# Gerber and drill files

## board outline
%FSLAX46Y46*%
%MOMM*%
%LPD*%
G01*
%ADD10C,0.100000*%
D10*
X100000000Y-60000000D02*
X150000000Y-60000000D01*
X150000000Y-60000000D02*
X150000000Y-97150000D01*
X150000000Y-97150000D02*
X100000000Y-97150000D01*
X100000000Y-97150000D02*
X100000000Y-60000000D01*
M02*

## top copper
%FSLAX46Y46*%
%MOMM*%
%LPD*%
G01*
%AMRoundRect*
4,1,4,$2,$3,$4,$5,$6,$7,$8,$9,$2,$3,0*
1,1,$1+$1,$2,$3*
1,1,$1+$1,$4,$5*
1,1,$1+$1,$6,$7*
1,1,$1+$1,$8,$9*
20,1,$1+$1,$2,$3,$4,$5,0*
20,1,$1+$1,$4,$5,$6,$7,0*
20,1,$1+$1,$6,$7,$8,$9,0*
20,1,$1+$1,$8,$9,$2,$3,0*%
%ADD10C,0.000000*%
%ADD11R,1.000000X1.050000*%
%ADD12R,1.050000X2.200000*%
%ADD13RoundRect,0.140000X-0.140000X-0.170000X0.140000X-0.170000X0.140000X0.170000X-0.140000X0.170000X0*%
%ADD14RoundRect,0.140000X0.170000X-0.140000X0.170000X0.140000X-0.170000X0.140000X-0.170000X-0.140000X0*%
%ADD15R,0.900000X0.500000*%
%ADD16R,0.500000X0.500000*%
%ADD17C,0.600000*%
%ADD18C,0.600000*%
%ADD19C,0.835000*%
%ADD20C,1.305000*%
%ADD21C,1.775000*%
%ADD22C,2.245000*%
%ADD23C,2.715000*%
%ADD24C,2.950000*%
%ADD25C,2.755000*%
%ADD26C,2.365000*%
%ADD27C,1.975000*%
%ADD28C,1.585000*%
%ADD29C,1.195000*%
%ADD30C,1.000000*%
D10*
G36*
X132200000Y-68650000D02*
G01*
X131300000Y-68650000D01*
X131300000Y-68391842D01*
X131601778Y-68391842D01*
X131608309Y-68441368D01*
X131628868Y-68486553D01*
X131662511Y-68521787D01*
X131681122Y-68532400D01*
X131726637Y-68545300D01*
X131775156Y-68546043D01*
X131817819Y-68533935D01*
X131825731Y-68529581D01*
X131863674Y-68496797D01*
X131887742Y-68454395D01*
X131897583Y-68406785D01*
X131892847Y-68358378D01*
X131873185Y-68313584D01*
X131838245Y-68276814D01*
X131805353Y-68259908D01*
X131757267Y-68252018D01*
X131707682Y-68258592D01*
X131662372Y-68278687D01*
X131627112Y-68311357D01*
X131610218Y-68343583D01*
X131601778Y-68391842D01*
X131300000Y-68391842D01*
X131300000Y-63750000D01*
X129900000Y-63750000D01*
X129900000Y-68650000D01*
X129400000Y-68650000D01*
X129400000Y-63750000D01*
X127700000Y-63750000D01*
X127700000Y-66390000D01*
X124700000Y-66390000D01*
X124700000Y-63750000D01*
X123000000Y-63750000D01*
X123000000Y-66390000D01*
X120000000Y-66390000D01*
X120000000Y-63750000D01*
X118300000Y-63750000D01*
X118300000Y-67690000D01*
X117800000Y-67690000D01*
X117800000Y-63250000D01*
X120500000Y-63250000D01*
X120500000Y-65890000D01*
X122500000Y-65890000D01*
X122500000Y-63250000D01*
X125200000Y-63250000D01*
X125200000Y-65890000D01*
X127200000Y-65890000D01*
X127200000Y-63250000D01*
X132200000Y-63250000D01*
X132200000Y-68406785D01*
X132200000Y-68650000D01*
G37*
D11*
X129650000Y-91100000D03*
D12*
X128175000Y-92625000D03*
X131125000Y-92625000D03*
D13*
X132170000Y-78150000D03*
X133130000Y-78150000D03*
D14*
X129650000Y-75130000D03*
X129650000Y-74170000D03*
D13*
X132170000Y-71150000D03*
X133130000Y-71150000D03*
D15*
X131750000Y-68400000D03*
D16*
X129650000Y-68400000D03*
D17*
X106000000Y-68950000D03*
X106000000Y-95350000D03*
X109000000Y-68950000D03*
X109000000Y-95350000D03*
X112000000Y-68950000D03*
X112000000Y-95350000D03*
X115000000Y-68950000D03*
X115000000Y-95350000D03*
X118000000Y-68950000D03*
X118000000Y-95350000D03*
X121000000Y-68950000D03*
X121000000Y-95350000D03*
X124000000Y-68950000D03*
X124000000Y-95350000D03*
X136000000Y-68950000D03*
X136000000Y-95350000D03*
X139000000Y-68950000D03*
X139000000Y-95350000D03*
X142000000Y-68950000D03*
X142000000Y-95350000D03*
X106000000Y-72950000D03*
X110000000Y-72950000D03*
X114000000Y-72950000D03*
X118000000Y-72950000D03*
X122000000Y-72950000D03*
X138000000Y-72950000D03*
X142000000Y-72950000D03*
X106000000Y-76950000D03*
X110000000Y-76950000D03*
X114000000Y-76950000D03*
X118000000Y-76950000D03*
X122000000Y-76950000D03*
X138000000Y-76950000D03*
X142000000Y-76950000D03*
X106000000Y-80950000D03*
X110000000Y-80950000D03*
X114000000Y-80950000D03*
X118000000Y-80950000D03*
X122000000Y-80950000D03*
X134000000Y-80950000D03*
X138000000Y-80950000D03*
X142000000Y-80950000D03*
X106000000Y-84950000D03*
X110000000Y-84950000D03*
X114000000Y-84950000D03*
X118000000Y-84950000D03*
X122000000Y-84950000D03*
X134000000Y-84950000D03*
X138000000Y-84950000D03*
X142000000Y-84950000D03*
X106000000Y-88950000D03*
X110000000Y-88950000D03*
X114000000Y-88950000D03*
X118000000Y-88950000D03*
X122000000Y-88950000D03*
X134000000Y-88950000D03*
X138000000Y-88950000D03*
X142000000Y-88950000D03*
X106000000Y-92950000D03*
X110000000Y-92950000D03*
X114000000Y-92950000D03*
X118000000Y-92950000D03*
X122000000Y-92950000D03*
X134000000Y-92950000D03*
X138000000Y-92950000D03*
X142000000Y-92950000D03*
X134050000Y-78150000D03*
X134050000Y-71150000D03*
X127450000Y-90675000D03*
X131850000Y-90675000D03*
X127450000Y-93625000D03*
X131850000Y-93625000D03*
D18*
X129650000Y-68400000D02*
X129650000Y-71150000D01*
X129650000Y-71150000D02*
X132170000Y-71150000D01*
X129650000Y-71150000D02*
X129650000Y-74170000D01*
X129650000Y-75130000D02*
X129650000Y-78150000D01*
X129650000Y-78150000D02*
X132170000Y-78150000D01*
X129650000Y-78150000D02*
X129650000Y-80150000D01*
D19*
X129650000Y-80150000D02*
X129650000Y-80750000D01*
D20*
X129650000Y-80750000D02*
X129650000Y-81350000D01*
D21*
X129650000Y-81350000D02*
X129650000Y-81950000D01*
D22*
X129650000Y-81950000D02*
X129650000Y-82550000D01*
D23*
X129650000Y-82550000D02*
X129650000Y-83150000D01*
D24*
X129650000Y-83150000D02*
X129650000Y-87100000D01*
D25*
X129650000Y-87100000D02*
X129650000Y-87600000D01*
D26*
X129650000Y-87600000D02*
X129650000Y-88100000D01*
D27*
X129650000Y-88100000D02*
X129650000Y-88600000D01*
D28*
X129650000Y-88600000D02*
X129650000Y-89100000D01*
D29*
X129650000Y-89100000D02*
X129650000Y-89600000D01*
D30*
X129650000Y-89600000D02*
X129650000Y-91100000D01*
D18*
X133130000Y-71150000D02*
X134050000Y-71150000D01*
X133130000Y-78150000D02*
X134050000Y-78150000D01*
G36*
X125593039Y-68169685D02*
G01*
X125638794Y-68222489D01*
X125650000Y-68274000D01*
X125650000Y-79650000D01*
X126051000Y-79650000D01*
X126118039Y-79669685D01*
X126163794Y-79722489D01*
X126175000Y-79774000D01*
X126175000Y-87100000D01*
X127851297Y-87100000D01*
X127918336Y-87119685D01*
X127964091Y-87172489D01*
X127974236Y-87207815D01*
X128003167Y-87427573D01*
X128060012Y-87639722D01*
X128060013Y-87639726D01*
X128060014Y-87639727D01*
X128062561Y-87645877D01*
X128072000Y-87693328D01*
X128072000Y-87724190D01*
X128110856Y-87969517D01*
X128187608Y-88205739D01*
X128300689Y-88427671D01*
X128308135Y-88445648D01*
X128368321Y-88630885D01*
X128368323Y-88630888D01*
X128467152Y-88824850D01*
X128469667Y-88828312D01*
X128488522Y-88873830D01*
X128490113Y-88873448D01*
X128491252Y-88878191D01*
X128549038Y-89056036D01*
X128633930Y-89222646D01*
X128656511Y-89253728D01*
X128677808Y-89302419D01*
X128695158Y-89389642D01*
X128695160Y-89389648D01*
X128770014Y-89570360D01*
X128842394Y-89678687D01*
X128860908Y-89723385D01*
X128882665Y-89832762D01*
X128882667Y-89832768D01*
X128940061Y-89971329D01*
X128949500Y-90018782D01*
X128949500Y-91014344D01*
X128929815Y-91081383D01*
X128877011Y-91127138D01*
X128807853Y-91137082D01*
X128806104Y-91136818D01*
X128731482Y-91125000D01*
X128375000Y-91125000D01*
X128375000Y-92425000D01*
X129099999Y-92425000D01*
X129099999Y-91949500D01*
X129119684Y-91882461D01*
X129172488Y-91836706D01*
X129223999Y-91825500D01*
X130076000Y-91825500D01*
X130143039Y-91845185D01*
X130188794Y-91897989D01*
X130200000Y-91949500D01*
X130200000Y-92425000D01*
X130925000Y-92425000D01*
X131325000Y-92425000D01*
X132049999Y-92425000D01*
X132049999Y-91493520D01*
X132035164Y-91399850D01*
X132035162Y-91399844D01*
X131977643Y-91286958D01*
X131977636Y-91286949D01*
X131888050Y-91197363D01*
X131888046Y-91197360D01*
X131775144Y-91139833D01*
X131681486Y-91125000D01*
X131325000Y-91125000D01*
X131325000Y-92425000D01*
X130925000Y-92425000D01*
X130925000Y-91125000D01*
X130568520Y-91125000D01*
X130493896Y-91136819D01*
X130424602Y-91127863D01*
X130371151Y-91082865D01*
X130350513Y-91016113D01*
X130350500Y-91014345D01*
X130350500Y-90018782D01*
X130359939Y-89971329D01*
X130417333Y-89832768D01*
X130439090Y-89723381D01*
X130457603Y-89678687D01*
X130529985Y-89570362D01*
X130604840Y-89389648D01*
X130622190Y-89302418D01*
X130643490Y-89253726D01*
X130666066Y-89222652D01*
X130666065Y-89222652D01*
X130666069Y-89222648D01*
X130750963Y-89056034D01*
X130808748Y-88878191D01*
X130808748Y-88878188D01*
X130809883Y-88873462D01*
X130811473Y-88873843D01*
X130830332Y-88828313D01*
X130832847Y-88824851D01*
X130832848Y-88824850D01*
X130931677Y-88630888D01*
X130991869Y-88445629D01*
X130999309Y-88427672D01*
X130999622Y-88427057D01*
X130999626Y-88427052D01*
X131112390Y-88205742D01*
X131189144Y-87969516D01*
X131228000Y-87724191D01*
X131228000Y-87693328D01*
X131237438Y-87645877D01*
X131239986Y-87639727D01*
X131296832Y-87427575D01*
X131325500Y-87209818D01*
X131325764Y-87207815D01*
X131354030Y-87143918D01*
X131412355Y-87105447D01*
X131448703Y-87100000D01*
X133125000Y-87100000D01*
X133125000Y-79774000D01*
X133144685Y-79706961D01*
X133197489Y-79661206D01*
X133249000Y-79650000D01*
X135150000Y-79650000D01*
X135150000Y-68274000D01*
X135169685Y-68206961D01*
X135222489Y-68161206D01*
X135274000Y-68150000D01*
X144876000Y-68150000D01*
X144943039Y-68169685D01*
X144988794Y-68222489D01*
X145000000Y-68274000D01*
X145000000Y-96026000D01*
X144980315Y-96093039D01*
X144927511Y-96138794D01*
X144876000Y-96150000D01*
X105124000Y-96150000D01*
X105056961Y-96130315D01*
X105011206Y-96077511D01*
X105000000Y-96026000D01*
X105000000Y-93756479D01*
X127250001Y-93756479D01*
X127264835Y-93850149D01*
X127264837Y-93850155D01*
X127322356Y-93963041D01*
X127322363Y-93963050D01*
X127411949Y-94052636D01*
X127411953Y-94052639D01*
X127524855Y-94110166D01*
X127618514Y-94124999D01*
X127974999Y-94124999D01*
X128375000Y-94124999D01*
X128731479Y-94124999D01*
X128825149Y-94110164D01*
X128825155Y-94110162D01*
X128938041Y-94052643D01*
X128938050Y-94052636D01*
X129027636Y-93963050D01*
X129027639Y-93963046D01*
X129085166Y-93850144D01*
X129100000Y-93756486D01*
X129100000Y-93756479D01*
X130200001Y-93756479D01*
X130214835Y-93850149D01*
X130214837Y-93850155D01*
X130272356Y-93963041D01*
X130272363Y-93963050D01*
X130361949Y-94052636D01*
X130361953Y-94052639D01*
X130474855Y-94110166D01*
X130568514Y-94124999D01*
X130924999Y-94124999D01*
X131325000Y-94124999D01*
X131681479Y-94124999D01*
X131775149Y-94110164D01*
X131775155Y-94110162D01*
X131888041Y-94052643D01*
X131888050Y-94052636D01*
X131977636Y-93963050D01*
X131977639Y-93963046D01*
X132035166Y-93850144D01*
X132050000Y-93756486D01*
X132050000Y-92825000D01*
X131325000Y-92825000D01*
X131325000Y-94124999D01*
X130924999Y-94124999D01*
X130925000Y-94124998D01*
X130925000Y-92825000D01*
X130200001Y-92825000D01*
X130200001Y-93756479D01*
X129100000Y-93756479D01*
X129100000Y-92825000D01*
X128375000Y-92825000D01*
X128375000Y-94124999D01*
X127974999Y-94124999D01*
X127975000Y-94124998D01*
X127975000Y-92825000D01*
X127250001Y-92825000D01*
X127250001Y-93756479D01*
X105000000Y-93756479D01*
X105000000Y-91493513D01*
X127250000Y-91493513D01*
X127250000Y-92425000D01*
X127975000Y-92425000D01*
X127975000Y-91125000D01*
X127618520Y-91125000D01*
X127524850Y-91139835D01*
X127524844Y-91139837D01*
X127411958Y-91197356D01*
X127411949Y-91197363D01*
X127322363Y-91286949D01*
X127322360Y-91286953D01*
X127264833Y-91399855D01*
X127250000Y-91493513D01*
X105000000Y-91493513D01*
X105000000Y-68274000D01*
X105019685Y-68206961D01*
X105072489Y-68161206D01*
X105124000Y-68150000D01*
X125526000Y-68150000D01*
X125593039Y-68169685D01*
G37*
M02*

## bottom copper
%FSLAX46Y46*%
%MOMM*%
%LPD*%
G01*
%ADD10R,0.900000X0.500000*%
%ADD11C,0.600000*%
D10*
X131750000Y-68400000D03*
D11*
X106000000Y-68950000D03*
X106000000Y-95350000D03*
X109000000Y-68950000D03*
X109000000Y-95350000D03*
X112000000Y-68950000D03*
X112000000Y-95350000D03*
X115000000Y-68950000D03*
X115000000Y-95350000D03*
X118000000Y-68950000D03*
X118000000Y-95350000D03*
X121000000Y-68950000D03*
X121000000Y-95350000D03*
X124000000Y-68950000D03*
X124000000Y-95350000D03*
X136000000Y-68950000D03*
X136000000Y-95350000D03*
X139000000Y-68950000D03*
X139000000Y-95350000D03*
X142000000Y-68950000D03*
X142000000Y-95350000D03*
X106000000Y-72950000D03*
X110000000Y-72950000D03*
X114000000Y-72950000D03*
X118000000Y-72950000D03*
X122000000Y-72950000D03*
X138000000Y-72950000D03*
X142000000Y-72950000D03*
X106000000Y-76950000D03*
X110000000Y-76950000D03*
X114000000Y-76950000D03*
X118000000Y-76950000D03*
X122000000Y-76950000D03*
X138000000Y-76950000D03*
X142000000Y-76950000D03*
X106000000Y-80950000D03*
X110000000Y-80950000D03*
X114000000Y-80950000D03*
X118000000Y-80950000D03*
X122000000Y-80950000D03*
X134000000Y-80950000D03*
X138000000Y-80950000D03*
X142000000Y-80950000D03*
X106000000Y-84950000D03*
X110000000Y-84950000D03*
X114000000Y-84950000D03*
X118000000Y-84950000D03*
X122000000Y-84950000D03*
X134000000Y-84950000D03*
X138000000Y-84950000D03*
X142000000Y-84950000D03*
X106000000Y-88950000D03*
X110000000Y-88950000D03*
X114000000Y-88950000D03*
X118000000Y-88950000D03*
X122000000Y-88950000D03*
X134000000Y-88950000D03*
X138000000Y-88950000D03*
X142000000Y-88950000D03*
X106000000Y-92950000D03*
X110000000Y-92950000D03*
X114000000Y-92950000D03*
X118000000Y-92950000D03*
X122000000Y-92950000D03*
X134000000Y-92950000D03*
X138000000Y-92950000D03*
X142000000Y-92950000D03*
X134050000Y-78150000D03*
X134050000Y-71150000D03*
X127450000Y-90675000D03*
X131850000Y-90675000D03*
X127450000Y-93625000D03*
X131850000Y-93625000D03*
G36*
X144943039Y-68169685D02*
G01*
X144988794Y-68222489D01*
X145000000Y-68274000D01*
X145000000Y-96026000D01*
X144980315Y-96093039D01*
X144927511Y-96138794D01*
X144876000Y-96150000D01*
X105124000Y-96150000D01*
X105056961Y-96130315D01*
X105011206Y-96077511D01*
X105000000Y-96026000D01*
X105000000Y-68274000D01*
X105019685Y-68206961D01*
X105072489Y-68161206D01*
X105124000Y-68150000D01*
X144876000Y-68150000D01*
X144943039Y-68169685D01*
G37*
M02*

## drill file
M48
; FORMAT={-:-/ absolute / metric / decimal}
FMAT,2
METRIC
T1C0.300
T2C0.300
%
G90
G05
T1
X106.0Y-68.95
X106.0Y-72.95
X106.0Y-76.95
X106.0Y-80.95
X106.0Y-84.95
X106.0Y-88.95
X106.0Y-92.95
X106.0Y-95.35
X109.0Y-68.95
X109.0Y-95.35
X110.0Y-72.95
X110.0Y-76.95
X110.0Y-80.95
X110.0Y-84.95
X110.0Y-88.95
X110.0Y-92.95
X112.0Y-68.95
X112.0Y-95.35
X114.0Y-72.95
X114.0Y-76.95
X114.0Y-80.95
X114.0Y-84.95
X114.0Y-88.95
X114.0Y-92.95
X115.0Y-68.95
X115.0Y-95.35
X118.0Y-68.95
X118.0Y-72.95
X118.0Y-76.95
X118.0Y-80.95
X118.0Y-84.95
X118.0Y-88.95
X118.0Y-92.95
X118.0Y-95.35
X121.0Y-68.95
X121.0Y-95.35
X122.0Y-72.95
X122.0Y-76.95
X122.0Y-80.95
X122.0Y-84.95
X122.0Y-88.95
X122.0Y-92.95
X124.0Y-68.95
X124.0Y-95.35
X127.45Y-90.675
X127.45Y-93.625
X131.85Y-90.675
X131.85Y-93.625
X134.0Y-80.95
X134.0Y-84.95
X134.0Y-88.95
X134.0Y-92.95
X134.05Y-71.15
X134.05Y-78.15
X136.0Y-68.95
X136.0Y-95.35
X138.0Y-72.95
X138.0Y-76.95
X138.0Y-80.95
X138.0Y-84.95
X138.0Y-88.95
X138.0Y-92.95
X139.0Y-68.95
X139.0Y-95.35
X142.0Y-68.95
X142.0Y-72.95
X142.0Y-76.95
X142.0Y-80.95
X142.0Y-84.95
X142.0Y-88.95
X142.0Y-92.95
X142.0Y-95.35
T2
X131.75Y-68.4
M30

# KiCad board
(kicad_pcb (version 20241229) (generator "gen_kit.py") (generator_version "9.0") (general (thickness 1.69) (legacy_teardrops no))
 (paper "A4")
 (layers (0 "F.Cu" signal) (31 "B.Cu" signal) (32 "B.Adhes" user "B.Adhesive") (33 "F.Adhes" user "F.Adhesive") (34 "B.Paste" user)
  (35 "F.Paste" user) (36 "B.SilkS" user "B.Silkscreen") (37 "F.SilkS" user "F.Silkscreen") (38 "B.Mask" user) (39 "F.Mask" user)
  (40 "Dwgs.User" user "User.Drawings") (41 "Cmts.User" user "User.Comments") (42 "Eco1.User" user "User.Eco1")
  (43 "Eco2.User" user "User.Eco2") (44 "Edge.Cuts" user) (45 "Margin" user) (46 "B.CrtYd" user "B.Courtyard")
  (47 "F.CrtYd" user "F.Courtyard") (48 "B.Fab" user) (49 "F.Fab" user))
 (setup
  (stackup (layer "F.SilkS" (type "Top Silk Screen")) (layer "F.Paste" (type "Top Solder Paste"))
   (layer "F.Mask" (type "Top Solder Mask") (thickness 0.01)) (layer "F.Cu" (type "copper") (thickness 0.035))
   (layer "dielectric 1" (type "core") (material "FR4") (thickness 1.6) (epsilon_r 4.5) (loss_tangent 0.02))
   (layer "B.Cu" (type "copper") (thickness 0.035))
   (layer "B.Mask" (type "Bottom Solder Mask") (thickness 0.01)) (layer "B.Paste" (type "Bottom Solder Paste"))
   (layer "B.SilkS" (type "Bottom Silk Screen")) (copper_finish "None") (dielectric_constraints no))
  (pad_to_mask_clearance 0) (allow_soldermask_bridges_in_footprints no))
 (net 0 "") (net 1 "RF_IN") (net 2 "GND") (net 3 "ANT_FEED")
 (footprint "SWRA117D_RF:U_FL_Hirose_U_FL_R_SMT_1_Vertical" (layer "F.Cu") (at 129.65 92.15 270)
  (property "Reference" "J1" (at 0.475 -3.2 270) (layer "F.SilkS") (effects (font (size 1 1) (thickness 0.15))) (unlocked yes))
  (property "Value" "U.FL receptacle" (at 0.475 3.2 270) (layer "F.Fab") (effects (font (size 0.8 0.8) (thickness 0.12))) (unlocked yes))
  (pad "1" smd rect (at -1.05 0 270) (size 1.05 1) (layers "F.Cu" "F.Paste" "F.Mask") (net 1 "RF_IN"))
  (pad "2" smd rect (at 0.475 1.475 270) (size 2.2 1.05) (layers "F.Cu" "F.Paste" "F.Mask") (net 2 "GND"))
  (pad "2" smd rect (at 0.475 -1.475 270) (size 2.2 1.05) (layers "F.Cu" "F.Paste" "F.Mask") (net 2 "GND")))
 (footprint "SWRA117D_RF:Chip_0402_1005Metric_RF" (layer "F.Cu") (at 132.65 78.15)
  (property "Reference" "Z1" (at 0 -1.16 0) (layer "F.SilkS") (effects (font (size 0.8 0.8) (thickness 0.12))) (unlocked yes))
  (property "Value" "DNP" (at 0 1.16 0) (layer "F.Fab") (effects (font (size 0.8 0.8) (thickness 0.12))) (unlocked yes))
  (pad "1" smd roundrect (at -0.48 0) (size 0.56 0.62) (layers "F.Cu" "F.Paste" "F.Mask") (roundrect_rratio 0.25) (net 1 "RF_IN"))
  (pad "2" smd roundrect (at 0.48 0) (size 0.56 0.62) (layers "F.Cu" "F.Paste" "F.Mask") (roundrect_rratio 0.25) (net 2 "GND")))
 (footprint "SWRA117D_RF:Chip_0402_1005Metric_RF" (layer "F.Cu") (at 129.65 74.65 90)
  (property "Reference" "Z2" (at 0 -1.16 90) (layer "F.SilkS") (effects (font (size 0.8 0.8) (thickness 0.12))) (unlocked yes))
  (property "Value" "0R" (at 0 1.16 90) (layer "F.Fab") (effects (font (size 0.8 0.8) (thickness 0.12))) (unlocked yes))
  (pad "1" smd roundrect (at -0.48 0 90) (size 0.56 0.62) (layers "F.Cu" "F.Paste" "F.Mask") (roundrect_rratio 0.25) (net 1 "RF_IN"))
  (pad "2" smd roundrect (at 0.48 0 90) (size 0.56 0.62) (layers "F.Cu" "F.Paste" "F.Mask") (roundrect_rratio 0.25) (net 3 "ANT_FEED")))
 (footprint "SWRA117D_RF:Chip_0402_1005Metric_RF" (layer "F.Cu") (at 132.65 71.15)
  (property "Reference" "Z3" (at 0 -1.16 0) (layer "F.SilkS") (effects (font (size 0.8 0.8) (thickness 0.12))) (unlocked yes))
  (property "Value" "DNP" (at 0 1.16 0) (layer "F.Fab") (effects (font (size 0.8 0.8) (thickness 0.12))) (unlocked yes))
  (pad "1" smd roundrect (at -0.48 0) (size 0.56 0.62) (layers "F.Cu" "F.Paste" "F.Mask") (roundrect_rratio 0.25) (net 3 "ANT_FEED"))
  (pad "2" smd roundrect (at 0.48 0) (size 0.56 0.62) (layers "F.Cu" "F.Paste" "F.Mask") (roundrect_rratio 0.25) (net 2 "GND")))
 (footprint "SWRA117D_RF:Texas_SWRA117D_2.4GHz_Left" (layer "F.Cu") (at 129.65 68.4)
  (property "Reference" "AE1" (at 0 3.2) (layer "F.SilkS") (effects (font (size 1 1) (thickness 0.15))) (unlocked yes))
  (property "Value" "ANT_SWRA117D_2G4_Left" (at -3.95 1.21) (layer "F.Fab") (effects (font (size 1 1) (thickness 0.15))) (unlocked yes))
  (fp_poly
   (pts (xy -2.45 -2.51) (xy -4.45 -2.51) (xy -4.45 -5.15) (xy -7.15 -5.15) (xy -7.15 -2.51) (xy -9.15 -2.51) (xy -9.15 -5.15)
    (xy -11.85 -5.15) (xy -11.85 -0.71) (xy -11.35 -0.71) (xy -11.35 -4.65) (xy -9.65 -4.65) (xy -9.65 -2.01) (xy -6.65 -2.01)
    (xy -6.65 -4.65) (xy -4.95 -4.65) (xy -4.95 -2.01) (xy -1.95 -2.01) (xy -1.95 -4.65) (xy -0.25 -4.65) (xy -0.25 0.25) (xy 0.25 0.25)
    (xy 0.25 -4.65) (xy 1.65 -4.65) (xy 1.65 0.25) (xy 2.55 0.25) (xy 2.55 0.006785) (xy 2.247583 0.006785) (xy 2.237742 0.054395)
    (xy 2.213674 0.096797) (xy 2.175731 0.129581) (xy 2.167819 0.133935) (xy 2.125156 0.146043) (xy 2.076637 0.1453) (xy 2.031122 0.1324)
    (xy 2.012511 0.121787) (xy 1.978868 0.086553) (xy 1.958309 0.041368) (xy 1.951778 -0.008158) (xy 1.960218 -0.056417)
    (xy 1.977112 -0.088643) (xy 2.012372 -0.121313) (xy 2.057682 -0.141408) (xy 2.107267 -0.147982) (xy 2.155353 -0.140092)
    (xy 2.188245 -0.123186) (xy 2.223185 -0.086416) (xy 2.242847 -0.041622) (xy 2.247583 0.006785) (xy 2.55 0.006785) (xy 2.55 -5.15)
    (xy -2.45 -5.15) (xy -2.45 -2.51))
   (stroke (width 0) (type solid)) (fill yes) (layer "F.Cu"))
  (pad "2" thru_hole rect (at 2.1 0) (size 0.9 0.5) (drill 0.3) (layers "*.Cu") (zone_connect 2) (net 2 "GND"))
  (pad "1" smd rect (at 0 0) (size 0.5 0.5) (layers "F.Cu") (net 3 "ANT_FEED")))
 (gr_line (start 100 60) (end 150 60) (stroke (width 0.1) (type solid)) (layer "Edge.Cuts"))
 (gr_line (start 150 60) (end 150 97.15) (stroke (width 0.1) (type solid)) (layer "Edge.Cuts"))
 (gr_line (start 150 97.15) (end 100 97.15) (stroke (width 0.1) (type solid)) (layer "Edge.Cuts"))
 (gr_line (start 100 97.15) (end 100 60) (stroke (width 0.1) (type solid)) (layer "Edge.Cuts"))
 (segment (start 129.65 68.4) (end 129.65 71.15) (width 0.6) (layer "F.Cu") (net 3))
 (segment (start 129.65 71.15) (end 132.17 71.15) (width 0.6) (layer "F.Cu") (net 3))
 (segment (start 129.65 71.15) (end 129.65 74.17) (width 0.6) (layer "F.Cu") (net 3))
 (segment (start 129.65 75.13) (end 129.65 78.15) (width 0.6) (layer "F.Cu") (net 1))
 (segment (start 129.65 78.15) (end 132.17 78.15) (width 0.6) (layer "F.Cu") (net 1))
 (segment (start 129.65 78.15) (end 129.65 80.15) (width 0.6) (layer "F.Cu") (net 1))
 (segment (start 129.65 80.15) (end 129.65 80.75) (width 0.835) (layer "F.Cu") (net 1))
 (segment (start 129.65 80.75) (end 129.65 81.35) (width 1.305) (layer "F.Cu") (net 1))
 (segment (start 129.65 81.35) (end 129.65 81.95) (width 1.775) (layer "F.Cu") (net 1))
 (segment (start 129.65 81.95) (end 129.65 82.55) (width 2.245) (layer "F.Cu") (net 1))
 (segment (start 129.65 82.55) (end 129.65 83.15) (width 2.715) (layer "F.Cu") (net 1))
 (segment (start 129.65 83.15) (end 129.65 87.1) (width 2.95) (layer "F.Cu") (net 1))
 (segment (start 129.65 87.1) (end 129.65 87.6) (width 2.755) (layer "F.Cu") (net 1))
 (segment (start 129.65 87.6) (end 129.65 88.1) (width 2.365) (layer "F.Cu") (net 1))
 (segment (start 129.65 88.1) (end 129.65 88.6) (width 1.975) (layer "F.Cu") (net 1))
 (segment (start 129.65 88.6) (end 129.65 89.1) (width 1.585) (layer "F.Cu") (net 1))
 (segment (start 129.65 89.1) (end 129.65 89.6) (width 1.195) (layer "F.Cu") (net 1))
 (segment (start 129.65 89.6) (end 129.65 91.1) (width 1) (layer "F.Cu") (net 1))
 (segment (start 133.13 71.15) (end 134.05 71.15) (width 0.6) (layer "F.Cu") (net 2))
 (segment (start 133.13 78.15) (end 134.05 78.15) (width 0.6) (layer "F.Cu") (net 2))
 (via (at 106 68.95) (size 0.6) (drill 0.3) (layers "F.Cu" "B.Cu") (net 2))
 (via (at 106 95.35) (size 0.6) (drill 0.3) (layers "F.Cu" "B.Cu") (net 2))
 (via (at 109 68.95) (size 0.6) (drill 0.3) (layers "F.Cu" "B.Cu") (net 2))
 (via (at 109 95.35) (size 0.6) (drill 0.3) (layers "F.Cu" "B.Cu") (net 2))
 (via (at 112 68.95) (size 0.6) (drill 0.3) (layers "F.Cu" "B.Cu") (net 2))
 (via (at 112 95.35) (size 0.6) (drill 0.3) (layers "F.Cu" "B.Cu") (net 2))
 (via (at 115 68.95) (size 0.6) (drill 0.3) (layers "F.Cu" "B.Cu") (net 2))
 (via (at 115 95.35) (size 0.6) (drill 0.3) (layers "F.Cu" "B.Cu") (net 2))
 (via (at 118 68.95) (size 0.6) (drill 0.3) (layers "F.Cu" "B.Cu") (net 2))
 (via (at 118 95.35) (size 0.6) (drill 0.3) (layers "F.Cu" "B.Cu") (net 2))
 (via (at 121 68.95) (size 0.6) (drill 0.3) (layers "F.Cu" "B.Cu") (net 2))
 (via (at 121 95.35) (size 0.6) (drill 0.3) (layers "F.Cu" "B.Cu") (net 2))
 (via (at 124 68.95) (size 0.6) (drill 0.3) (layers "F.Cu" "B.Cu") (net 2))
 (via (at 124 95.35) (size 0.6) (drill 0.3) (layers "F.Cu" "B.Cu") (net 2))
 (via (at 136 68.95) (size 0.6) (drill 0.3) (layers "F.Cu" "B.Cu") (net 2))
 (via (at 136 95.35) (size 0.6) (drill 0.3) (layers "F.Cu" "B.Cu") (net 2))
 (via (at 139 68.95) (size 0.6) (drill 0.3) (layers "F.Cu" "B.Cu") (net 2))
 (via (at 139 95.35) (size 0.6) (drill 0.3) (layers "F.Cu" "B.Cu") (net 2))
 (via (at 142 68.95) (size 0.6) (drill 0.3) (layers "F.Cu" "B.Cu") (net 2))
 (via (at 142 95.35) (size 0.6) (drill 0.3) (layers "F.Cu" "B.Cu") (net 2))
 (via (at 106 72.95) (size 0.6) (drill 0.3) (layers "F.Cu" "B.Cu") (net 2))
 (via (at 110 72.95) (size 0.6) (drill 0.3) (layers "F.Cu" "B.Cu") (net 2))
 (via (at 114 72.95) (size 0.6) (drill 0.3) (layers "F.Cu" "B.Cu") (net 2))
 (via (at 118 72.95) (size 0.6) (drill 0.3) (layers "F.Cu" "B.Cu") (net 2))
 (via (at 122 72.95) (size 0.6) (drill 0.3) (layers "F.Cu" "B.Cu") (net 2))
 (via (at 138 72.95) (size 0.6) (drill 0.3) (layers "F.Cu" "B.Cu") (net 2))
 (via (at 142 72.95) (size 0.6) (drill 0.3) (layers "F.Cu" "B.Cu") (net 2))
 (via (at 106 76.95) (size 0.6) (drill 0.3) (layers "F.Cu" "B.Cu") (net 2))
 (via (at 110 76.95) (size 0.6) (drill 0.3) (layers "F.Cu" "B.Cu") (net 2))
 (via (at 114 76.95) (size 0.6) (drill 0.3) (layers "F.Cu" "B.Cu") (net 2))
 (via (at 118 76.95) (size 0.6) (drill 0.3) (layers "F.Cu" "B.Cu") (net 2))
 (via (at 122 76.95) (size 0.6) (drill 0.3) (layers "F.Cu" "B.Cu") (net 2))
 (via (at 138 76.95) (size 0.6) (drill 0.3) (layers "F.Cu" "B.Cu") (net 2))
 (via (at 142 76.95) (size 0.6) (drill 0.3) (layers "F.Cu" "B.Cu") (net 2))
 (via (at 106 80.95) (size 0.6) (drill 0.3) (layers "F.Cu" "B.Cu") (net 2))
 (via (at 110 80.95) (size 0.6) (drill 0.3) (layers "F.Cu" "B.Cu") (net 2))
 (via (at 114 80.95) (size 0.6) (drill 0.3) (layers "F.Cu" "B.Cu") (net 2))
 (via (at 118 80.95) (size 0.6) (drill 0.3) (layers "F.Cu" "B.Cu") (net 2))
 (via (at 122 80.95) (size 0.6) (drill 0.3) (layers "F.Cu" "B.Cu") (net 2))
 (via (at 134 80.95) (size 0.6) (drill 0.3) (layers "F.Cu" "B.Cu") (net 2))
 (via (at 138 80.95) (size 0.6) (drill 0.3) (layers "F.Cu" "B.Cu") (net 2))
 (via (at 142 80.95) (size 0.6) (drill 0.3) (layers "F.Cu" "B.Cu") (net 2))
 (via (at 106 84.95) (size 0.6) (drill 0.3) (layers "F.Cu" "B.Cu") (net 2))
 (via (at 110 84.95) (size 0.6) (drill 0.3) (layers "F.Cu" "B.Cu") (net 2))
 (via (at 114 84.95) (size 0.6) (drill 0.3) (layers "F.Cu" "B.Cu") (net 2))
 (via (at 118 84.95) (size 0.6) (drill 0.3) (layers "F.Cu" "B.Cu") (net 2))
 (via (at 122 84.95) (size 0.6) (drill 0.3) (layers "F.Cu" "B.Cu") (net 2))
 (via (at 134 84.95) (size 0.6) (drill 0.3) (layers "F.Cu" "B.Cu") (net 2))
 (via (at 138 84.95) (size 0.6) (drill 0.3) (layers "F.Cu" "B.Cu") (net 2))
 (via (at 142 84.95) (size 0.6) (drill 0.3) (layers "F.Cu" "B.Cu") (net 2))
 (via (at 106 88.95) (size 0.6) (drill 0.3) (layers "F.Cu" "B.Cu") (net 2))
 (via (at 110 88.95) (size 0.6) (drill 0.3) (layers "F.Cu" "B.Cu") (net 2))
 (via (at 114 88.95) (size 0.6) (drill 0.3) (layers "F.Cu" "B.Cu") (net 2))
 (via (at 118 88.95) (size 0.6) (drill 0.3) (layers "F.Cu" "B.Cu") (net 2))
 (via (at 122 88.95) (size 0.6) (drill 0.3) (layers "F.Cu" "B.Cu") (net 2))
 (via (at 134 88.95) (size 0.6) (drill 0.3) (layers "F.Cu" "B.Cu") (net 2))
 (via (at 138 88.95) (size 0.6) (drill 0.3) (layers "F.Cu" "B.Cu") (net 2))
 (via (at 142 88.95) (size 0.6) (drill 0.3) (layers "F.Cu" "B.Cu") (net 2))
 (via (at 106 92.95) (size 0.6) (drill 0.3) (layers "F.Cu" "B.Cu") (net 2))
 (via (at 110 92.95) (size 0.6) (drill 0.3) (layers "F.Cu" "B.Cu") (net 2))
 (via (at 114 92.95) (size 0.6) (drill 0.3) (layers "F.Cu" "B.Cu") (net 2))
 (via (at 118 92.95) (size 0.6) (drill 0.3) (layers "F.Cu" "B.Cu") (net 2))
 (via (at 122 92.95) (size 0.6) (drill 0.3) (layers "F.Cu" "B.Cu") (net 2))
 (via (at 134 92.95) (size 0.6) (drill 0.3) (layers "F.Cu" "B.Cu") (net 2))
 (via (at 138 92.95) (size 0.6) (drill 0.3) (layers "F.Cu" "B.Cu") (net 2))
 (via (at 142 92.95) (size 0.6) (drill 0.3) (layers "F.Cu" "B.Cu") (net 2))
 (via (at 134.05 78.15) (size 0.6) (drill 0.3) (layers "F.Cu" "B.Cu") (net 2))
 (via (at 134.05 71.15) (size 0.6) (drill 0.3) (layers "F.Cu" "B.Cu") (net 2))
 (via (at 127.45 90.675) (size 0.6) (drill 0.3) (layers "F.Cu" "B.Cu") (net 2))
 (via (at 131.85 90.675) (size 0.6) (drill 0.3) (layers "F.Cu" "B.Cu") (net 2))
 (via (at 127.45 93.625) (size 0.6) (drill 0.3) (layers "F.Cu" "B.Cu") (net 2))
 (via (at 131.85 93.625) (size 0.6) (drill 0.3) (layers "F.Cu" "B.Cu") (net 2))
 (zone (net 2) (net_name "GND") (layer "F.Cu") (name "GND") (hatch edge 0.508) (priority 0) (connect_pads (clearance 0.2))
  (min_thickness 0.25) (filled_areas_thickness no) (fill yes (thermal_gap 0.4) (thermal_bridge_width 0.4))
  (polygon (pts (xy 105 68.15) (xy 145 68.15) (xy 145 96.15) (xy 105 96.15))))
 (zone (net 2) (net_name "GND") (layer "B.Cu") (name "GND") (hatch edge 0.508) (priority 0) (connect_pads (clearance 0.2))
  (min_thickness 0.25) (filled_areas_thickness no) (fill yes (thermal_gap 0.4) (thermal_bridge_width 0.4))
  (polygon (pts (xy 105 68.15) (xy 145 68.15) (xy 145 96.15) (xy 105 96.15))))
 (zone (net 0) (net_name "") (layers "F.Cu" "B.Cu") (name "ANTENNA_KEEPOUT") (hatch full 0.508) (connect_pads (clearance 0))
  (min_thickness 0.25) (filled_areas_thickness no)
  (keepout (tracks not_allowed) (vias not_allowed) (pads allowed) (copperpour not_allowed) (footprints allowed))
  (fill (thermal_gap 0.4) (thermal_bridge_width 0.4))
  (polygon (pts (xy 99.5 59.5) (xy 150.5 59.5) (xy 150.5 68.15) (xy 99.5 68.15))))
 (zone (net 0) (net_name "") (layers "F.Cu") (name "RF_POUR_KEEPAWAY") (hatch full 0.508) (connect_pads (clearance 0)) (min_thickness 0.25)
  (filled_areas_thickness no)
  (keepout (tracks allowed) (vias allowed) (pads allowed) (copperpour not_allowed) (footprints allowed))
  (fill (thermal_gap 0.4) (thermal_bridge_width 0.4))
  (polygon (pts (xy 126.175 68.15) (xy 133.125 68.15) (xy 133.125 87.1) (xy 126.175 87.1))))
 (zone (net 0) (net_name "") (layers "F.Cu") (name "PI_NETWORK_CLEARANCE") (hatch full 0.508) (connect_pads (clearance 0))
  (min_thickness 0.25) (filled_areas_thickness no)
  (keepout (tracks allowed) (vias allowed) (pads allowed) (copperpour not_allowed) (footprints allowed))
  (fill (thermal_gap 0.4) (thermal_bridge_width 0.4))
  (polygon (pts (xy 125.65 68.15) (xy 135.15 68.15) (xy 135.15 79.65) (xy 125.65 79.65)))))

